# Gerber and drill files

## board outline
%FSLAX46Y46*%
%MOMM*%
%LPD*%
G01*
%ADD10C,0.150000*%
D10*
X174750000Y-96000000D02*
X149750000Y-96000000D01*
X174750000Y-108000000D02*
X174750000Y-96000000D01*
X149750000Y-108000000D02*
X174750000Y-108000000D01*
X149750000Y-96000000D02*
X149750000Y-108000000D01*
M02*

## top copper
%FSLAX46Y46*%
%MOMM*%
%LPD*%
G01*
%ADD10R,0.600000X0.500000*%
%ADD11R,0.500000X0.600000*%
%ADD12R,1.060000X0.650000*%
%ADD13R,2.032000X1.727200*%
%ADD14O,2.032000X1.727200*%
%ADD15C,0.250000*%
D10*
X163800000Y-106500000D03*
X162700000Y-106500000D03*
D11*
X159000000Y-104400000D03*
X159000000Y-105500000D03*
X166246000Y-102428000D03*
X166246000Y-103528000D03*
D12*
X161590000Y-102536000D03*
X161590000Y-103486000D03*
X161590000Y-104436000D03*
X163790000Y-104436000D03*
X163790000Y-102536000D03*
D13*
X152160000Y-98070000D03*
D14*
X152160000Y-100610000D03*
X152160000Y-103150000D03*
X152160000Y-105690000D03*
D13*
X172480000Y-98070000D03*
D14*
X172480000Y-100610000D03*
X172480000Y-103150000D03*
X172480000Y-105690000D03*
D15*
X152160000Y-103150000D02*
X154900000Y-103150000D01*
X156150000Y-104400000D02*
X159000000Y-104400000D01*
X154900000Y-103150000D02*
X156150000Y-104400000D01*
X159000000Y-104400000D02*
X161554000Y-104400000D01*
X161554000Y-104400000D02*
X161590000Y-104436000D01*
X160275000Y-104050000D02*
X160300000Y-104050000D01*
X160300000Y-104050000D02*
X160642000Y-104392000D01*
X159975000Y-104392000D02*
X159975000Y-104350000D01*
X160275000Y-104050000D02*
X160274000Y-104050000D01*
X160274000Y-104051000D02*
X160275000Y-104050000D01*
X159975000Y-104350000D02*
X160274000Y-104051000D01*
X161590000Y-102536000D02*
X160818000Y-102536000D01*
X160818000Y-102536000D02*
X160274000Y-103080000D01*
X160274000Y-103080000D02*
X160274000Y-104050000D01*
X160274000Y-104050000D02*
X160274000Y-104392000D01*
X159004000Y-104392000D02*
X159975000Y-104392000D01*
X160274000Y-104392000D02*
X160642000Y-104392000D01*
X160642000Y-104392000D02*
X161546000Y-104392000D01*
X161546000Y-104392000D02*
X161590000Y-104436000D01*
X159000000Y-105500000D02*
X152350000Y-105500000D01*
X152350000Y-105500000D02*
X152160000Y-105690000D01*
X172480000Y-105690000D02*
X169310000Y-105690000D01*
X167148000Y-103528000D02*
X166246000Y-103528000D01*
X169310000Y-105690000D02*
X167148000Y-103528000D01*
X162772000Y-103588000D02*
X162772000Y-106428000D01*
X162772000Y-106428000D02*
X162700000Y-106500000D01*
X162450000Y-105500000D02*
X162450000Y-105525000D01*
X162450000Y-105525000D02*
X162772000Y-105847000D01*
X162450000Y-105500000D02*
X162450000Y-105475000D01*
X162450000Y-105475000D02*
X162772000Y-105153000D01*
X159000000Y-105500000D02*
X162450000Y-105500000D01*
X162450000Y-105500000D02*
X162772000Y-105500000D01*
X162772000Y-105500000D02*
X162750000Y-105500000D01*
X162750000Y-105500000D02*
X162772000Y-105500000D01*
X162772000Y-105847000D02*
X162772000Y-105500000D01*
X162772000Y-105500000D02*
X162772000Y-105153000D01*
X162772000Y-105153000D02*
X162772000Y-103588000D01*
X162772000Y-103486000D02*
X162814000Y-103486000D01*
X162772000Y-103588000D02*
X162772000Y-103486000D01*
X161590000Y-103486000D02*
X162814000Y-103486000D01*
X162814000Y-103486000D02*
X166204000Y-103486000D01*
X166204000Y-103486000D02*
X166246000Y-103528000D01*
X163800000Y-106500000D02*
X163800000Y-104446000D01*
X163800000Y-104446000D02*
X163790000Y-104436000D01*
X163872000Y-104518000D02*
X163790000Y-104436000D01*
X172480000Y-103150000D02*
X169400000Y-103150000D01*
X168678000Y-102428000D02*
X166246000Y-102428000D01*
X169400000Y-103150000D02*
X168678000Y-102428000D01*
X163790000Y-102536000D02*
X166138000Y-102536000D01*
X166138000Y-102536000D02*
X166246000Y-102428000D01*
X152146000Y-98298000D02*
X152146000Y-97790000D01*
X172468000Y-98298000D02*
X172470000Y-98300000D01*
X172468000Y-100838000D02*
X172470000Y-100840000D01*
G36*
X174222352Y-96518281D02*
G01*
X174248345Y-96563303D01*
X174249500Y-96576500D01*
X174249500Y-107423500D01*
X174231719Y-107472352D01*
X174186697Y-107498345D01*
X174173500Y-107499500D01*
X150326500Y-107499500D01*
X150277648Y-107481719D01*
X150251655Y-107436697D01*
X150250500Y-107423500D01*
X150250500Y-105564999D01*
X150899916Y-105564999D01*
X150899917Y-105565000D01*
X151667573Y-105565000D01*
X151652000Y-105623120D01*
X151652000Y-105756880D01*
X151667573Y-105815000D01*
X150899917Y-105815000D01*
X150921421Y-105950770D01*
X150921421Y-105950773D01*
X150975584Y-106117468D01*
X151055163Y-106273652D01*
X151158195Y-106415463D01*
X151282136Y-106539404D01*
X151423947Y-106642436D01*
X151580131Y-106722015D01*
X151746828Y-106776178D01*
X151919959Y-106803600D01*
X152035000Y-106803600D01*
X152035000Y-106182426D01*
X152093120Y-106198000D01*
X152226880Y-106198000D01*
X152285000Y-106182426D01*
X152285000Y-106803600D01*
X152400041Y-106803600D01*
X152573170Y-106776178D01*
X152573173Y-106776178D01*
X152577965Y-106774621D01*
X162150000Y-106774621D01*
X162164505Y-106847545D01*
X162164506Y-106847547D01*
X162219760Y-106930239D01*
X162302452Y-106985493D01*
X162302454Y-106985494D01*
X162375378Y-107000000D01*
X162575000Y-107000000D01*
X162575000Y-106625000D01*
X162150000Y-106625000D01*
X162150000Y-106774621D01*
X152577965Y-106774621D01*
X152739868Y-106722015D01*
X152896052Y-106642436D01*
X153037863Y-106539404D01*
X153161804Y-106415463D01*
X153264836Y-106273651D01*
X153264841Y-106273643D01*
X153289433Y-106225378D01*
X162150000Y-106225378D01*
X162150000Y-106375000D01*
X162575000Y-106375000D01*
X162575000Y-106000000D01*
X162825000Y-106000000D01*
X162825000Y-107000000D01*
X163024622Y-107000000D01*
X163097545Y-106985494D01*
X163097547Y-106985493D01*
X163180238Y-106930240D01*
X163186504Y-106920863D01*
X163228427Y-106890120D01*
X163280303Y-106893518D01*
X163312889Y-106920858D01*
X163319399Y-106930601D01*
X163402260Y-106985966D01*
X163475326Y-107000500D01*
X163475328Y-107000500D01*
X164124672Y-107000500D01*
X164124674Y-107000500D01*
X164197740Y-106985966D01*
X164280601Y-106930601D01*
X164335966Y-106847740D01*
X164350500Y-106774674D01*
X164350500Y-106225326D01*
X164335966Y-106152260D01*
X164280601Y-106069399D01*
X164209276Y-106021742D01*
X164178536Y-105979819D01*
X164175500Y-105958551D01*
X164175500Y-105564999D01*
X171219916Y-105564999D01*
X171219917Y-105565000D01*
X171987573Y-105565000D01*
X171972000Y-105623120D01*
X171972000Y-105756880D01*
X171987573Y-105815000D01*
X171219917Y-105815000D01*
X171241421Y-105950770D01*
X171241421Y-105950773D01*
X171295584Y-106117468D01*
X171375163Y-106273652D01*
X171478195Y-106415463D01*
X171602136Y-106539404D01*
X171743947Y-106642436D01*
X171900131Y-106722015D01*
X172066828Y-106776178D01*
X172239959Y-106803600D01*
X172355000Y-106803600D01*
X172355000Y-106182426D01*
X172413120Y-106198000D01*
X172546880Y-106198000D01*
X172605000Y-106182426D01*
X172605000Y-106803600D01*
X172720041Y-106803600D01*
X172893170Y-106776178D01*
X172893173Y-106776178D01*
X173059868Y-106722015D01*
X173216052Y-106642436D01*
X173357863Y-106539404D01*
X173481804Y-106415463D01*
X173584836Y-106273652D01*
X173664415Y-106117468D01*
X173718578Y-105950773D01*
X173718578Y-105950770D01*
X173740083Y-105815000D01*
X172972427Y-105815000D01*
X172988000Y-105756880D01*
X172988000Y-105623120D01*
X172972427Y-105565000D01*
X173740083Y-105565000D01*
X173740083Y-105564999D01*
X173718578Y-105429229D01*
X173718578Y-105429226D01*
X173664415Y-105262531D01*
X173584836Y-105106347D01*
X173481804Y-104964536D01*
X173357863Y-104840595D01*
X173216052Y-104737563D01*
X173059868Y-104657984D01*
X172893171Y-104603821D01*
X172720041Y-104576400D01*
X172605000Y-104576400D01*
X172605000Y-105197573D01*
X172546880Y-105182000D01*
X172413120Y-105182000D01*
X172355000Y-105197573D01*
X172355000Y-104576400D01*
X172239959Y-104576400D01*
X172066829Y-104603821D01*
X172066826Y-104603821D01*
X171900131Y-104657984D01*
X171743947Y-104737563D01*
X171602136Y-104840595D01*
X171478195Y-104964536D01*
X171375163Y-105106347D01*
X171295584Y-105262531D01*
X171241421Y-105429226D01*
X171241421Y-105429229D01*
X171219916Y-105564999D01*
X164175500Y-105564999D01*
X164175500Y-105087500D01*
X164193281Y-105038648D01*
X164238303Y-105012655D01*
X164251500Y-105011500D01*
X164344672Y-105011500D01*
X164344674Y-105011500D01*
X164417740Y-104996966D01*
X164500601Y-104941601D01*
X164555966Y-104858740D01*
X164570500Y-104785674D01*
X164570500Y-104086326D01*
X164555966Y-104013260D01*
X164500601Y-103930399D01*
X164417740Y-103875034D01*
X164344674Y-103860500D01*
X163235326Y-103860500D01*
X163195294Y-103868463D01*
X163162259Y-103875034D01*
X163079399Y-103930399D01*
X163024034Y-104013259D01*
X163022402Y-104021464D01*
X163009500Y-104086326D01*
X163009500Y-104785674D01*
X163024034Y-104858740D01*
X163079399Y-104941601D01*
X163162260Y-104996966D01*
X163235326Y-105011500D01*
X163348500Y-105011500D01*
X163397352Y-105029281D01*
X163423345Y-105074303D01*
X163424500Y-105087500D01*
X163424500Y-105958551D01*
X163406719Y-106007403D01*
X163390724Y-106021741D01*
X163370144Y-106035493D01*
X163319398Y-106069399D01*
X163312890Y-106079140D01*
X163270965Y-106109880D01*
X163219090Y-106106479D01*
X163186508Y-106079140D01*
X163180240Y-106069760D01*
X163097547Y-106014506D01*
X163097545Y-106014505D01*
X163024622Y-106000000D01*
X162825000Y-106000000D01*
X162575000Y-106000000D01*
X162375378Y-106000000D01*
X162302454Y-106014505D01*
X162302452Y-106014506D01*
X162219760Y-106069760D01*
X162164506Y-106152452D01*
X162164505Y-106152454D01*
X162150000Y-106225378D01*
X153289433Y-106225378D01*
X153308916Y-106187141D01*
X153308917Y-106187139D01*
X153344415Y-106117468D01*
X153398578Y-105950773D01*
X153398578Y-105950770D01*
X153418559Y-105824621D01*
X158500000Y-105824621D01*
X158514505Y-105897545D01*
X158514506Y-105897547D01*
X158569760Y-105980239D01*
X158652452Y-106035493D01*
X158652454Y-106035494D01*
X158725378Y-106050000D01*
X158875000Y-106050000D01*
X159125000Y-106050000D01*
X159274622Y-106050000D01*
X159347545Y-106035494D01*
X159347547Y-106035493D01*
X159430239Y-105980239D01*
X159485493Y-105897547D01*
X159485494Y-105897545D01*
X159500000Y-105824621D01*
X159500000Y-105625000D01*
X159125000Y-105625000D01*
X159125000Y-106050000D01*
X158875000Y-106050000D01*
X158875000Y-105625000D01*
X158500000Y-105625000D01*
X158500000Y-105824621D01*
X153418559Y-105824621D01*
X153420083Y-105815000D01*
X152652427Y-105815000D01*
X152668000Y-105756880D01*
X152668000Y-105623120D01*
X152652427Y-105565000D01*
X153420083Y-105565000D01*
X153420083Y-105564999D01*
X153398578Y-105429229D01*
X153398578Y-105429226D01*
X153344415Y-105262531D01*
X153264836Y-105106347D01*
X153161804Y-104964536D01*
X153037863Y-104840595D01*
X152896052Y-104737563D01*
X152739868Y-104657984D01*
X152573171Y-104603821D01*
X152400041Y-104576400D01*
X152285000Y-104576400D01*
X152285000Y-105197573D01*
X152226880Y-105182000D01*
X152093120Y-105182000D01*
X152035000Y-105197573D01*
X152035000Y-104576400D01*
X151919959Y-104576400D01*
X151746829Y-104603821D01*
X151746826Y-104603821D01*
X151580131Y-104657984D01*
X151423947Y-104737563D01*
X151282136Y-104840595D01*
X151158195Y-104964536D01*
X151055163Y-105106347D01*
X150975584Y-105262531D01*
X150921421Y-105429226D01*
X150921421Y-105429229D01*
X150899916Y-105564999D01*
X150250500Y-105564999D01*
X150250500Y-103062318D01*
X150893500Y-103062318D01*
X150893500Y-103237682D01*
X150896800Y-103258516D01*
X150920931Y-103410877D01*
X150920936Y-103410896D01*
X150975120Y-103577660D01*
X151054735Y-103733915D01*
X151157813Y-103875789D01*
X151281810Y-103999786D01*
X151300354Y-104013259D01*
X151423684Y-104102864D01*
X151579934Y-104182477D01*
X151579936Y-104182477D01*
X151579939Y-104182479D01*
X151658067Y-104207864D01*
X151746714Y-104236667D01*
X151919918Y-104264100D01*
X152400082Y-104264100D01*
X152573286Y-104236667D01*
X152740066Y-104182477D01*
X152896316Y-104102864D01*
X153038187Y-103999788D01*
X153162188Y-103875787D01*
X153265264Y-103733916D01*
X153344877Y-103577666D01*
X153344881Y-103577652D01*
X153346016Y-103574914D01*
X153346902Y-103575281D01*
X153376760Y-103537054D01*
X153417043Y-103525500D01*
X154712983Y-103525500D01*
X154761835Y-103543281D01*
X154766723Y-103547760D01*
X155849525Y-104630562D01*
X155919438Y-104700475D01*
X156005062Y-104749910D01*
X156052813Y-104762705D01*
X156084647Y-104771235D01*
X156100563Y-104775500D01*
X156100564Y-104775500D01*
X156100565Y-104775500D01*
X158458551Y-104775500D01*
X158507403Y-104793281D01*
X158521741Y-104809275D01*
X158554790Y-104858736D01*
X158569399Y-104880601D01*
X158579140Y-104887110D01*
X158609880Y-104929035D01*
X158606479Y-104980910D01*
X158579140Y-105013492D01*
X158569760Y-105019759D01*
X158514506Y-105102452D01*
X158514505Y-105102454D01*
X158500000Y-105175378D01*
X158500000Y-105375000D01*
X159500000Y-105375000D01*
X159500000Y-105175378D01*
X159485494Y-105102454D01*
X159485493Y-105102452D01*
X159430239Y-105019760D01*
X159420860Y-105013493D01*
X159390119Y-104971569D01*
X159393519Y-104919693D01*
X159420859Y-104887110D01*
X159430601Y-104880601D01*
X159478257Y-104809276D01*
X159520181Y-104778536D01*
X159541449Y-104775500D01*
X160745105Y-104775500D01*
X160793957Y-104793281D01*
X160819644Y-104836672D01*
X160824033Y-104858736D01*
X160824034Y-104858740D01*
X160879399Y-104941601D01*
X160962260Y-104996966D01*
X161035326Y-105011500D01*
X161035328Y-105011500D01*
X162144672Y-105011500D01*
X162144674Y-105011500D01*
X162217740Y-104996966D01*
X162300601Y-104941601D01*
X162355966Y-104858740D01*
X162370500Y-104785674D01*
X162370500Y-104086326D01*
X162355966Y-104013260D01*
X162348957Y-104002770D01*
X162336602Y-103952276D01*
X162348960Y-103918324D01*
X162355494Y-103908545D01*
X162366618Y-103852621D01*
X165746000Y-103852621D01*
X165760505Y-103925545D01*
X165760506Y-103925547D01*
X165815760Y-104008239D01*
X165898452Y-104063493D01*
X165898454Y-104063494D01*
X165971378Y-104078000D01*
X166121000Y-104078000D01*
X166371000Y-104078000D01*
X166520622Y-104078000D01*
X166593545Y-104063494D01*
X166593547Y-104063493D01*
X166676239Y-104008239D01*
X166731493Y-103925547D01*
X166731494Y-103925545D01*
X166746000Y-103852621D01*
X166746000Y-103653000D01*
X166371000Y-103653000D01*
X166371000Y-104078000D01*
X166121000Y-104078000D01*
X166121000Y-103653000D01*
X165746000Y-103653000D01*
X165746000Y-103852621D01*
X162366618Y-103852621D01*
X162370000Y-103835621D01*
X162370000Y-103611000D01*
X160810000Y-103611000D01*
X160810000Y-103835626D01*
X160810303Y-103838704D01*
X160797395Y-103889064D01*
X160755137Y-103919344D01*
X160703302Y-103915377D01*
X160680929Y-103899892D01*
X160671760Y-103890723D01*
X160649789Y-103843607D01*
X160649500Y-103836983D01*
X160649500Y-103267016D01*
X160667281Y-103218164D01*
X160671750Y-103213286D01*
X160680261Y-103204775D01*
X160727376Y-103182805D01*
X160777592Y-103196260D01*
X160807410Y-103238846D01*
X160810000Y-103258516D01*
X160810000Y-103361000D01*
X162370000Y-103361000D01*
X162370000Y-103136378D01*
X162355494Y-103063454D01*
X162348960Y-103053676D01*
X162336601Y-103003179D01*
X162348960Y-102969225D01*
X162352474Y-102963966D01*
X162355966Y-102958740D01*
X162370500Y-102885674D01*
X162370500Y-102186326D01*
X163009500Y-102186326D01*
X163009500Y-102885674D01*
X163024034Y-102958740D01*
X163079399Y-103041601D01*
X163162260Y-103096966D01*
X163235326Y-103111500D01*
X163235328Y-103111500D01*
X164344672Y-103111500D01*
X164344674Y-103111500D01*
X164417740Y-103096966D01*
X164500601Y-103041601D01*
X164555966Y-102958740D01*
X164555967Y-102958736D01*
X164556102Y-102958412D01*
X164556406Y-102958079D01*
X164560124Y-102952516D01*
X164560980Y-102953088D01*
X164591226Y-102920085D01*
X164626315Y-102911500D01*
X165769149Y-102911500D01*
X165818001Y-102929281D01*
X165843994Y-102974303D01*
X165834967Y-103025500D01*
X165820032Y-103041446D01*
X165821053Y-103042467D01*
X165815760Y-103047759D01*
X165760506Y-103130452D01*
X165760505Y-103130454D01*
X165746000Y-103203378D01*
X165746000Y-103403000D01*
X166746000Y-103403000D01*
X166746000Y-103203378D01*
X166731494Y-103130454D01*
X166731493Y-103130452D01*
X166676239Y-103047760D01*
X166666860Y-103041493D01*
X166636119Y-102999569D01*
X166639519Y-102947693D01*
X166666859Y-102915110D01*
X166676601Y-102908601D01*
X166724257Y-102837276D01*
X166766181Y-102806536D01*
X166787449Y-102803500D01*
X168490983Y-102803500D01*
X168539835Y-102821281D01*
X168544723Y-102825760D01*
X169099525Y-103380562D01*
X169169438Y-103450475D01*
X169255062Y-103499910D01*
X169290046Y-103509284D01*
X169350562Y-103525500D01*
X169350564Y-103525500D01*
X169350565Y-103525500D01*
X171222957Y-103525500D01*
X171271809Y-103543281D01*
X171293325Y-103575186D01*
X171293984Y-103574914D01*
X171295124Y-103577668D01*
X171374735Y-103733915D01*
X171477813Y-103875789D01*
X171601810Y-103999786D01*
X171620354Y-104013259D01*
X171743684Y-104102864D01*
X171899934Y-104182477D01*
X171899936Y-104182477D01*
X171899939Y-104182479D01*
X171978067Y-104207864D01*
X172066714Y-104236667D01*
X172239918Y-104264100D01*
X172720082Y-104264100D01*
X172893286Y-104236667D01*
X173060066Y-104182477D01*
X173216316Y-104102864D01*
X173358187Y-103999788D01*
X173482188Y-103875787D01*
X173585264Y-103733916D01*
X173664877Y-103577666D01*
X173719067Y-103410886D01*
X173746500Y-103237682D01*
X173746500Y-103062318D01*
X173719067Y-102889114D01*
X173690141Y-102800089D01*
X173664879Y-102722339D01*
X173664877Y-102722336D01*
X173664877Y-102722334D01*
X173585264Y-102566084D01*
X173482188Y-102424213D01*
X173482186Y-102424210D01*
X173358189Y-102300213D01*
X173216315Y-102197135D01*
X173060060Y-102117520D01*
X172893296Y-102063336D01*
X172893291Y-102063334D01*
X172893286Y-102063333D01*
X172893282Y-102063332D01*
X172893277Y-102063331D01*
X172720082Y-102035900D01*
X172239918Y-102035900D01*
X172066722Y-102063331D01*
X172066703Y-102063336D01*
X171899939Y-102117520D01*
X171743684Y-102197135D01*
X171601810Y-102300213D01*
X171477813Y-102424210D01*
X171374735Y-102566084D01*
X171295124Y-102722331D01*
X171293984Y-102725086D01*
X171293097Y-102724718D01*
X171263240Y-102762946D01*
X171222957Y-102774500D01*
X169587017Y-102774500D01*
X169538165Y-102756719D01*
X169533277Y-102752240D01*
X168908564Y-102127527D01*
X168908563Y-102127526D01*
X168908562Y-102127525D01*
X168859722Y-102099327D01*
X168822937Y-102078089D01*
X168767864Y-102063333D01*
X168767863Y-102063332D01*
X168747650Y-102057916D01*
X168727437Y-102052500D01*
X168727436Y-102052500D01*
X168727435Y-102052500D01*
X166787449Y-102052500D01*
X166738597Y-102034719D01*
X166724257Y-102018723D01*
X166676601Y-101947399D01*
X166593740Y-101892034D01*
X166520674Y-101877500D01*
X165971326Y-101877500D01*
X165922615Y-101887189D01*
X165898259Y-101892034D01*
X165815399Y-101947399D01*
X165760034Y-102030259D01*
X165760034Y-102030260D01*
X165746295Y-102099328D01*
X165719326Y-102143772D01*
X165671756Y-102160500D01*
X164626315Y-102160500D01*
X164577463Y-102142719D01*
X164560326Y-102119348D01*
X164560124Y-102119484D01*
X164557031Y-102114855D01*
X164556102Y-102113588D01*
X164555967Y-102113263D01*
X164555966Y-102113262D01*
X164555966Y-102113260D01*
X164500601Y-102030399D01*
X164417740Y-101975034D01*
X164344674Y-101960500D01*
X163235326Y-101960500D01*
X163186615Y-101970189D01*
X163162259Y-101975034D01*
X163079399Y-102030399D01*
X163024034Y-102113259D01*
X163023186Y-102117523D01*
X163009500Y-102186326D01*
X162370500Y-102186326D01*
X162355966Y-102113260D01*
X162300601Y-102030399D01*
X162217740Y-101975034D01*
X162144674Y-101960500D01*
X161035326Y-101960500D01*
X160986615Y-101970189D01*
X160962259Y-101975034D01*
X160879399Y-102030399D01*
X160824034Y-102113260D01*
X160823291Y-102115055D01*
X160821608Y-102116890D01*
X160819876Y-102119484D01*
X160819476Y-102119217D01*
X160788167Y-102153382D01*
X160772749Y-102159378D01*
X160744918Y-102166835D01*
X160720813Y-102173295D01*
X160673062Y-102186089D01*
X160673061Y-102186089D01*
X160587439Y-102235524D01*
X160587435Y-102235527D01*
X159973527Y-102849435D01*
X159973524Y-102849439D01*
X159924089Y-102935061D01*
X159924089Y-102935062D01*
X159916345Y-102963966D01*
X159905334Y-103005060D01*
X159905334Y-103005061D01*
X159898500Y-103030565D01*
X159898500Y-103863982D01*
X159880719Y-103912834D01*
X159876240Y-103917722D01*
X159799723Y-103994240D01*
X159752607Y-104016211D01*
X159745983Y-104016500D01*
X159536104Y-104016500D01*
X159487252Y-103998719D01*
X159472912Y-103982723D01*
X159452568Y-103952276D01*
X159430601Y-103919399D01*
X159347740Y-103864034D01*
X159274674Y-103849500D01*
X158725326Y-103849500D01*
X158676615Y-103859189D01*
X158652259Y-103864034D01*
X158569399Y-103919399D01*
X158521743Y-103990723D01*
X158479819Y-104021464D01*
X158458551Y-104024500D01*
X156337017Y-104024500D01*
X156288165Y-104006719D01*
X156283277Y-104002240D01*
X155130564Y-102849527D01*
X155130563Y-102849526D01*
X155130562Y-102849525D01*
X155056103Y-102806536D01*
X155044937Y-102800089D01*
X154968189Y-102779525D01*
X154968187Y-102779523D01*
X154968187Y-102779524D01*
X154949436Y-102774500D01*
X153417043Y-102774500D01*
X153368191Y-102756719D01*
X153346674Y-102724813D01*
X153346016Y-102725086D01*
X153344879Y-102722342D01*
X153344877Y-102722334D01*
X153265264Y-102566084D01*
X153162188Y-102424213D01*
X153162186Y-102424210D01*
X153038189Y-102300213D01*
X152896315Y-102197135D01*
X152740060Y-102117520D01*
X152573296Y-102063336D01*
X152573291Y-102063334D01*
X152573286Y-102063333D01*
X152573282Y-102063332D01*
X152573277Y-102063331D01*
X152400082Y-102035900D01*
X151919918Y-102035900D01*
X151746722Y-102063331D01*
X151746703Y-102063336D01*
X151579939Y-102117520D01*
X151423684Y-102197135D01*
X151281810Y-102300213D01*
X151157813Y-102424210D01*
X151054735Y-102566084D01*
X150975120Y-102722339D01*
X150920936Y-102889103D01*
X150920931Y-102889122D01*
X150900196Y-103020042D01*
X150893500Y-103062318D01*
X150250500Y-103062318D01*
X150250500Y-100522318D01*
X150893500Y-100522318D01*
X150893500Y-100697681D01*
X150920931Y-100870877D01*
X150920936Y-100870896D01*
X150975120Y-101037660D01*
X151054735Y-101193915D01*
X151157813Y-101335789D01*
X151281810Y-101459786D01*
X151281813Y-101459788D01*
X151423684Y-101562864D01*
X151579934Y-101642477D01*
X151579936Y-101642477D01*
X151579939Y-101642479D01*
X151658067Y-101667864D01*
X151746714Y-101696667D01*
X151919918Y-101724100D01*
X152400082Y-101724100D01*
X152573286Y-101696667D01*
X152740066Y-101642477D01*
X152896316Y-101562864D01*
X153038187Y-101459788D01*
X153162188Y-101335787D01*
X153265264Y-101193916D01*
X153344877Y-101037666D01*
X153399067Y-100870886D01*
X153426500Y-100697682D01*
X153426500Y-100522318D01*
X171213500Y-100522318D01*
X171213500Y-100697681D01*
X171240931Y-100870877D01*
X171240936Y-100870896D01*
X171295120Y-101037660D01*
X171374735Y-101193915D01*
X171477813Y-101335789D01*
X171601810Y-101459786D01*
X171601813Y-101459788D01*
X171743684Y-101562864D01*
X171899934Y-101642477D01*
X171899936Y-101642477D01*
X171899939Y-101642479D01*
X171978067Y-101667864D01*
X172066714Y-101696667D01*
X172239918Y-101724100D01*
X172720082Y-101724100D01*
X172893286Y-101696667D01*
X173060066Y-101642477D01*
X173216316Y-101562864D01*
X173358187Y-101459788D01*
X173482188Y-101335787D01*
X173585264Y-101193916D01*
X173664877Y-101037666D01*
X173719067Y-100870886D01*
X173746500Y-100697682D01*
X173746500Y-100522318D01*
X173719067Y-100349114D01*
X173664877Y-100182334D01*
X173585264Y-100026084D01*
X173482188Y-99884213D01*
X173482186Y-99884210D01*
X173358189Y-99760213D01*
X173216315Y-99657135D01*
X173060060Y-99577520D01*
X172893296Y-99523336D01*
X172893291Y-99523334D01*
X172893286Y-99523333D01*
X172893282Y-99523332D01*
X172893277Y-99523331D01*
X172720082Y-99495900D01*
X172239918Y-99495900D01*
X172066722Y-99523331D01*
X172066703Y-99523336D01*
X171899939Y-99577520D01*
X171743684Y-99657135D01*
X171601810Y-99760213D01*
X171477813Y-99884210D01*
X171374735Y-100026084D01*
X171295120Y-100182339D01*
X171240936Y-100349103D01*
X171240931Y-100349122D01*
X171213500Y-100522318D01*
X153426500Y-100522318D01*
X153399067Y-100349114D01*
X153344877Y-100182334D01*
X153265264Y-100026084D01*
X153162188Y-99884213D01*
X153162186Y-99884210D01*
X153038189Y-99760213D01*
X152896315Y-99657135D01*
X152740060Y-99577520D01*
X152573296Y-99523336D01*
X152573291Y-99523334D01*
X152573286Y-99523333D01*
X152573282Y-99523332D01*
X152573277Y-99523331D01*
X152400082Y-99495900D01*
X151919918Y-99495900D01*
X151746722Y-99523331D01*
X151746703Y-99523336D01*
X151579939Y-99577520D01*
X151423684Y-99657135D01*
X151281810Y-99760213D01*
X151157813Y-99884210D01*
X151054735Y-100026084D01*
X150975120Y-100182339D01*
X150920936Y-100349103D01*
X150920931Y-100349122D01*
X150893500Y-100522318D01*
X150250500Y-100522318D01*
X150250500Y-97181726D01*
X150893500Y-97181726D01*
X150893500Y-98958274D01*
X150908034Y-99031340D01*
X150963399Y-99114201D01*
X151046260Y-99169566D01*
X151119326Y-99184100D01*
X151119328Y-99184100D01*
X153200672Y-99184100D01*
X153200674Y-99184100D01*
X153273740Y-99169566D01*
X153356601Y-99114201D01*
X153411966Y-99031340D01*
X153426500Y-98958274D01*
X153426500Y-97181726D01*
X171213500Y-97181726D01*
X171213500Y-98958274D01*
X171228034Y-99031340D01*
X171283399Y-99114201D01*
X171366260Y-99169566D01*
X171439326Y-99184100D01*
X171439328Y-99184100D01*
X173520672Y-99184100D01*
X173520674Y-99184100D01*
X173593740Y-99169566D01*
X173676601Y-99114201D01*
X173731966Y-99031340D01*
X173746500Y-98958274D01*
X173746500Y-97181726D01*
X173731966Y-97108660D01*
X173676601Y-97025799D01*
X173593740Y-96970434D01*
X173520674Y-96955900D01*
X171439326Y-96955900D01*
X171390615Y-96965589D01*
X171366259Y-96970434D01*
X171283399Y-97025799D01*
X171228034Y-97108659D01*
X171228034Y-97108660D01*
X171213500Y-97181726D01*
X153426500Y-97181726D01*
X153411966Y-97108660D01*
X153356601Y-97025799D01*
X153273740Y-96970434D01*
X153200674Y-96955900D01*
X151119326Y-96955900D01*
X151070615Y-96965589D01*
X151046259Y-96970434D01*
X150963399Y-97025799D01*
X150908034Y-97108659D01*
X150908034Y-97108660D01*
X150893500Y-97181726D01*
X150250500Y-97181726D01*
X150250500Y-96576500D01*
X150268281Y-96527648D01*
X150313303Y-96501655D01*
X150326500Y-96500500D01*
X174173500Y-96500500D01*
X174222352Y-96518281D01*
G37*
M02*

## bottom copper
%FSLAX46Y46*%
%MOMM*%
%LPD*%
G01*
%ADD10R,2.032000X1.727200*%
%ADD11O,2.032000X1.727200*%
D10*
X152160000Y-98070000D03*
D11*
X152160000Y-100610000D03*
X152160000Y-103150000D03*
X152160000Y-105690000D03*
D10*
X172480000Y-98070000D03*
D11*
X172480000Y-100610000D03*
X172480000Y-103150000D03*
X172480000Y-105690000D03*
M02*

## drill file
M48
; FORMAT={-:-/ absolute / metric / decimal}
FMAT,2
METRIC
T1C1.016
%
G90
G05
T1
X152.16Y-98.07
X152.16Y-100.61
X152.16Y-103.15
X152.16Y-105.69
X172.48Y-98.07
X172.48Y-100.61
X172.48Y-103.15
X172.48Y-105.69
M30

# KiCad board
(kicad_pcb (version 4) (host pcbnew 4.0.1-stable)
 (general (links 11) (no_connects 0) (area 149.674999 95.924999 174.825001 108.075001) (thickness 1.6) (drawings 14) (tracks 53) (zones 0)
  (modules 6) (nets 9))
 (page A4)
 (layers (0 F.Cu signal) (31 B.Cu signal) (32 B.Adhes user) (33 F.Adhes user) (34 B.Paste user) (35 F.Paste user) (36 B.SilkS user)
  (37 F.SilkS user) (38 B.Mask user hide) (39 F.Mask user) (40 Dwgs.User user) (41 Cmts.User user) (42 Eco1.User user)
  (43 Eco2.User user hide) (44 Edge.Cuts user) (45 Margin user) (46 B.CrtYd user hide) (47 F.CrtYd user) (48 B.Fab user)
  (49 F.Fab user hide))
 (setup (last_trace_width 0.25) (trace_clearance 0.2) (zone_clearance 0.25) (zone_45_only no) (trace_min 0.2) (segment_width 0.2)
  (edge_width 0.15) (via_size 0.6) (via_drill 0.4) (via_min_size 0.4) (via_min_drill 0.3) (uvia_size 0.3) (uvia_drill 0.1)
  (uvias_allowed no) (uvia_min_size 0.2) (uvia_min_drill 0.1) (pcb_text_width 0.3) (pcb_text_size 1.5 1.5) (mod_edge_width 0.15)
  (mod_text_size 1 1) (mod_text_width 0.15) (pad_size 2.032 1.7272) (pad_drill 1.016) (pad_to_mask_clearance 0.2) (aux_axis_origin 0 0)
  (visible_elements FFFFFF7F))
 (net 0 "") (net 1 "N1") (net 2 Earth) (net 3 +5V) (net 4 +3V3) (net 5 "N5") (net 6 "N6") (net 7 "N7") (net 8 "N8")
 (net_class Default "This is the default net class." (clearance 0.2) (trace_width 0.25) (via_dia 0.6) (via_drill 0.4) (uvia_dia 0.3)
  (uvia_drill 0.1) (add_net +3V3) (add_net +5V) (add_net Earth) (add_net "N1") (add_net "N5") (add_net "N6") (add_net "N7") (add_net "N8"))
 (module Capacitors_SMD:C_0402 (layer F.Cu) (at 163.25 106.5 180)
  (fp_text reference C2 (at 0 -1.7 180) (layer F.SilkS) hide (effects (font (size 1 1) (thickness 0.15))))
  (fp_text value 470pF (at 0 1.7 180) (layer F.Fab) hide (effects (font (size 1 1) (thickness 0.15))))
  (pad 1 smd rect (at -0.55 0 180) (size 0.6 0.5) (layers F.Cu F.Paste F.Mask) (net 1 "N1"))
  (pad 2 smd rect (at 0.55 0 180) (size 0.6 0.5) (layers F.Cu F.Paste F.Mask) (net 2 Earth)))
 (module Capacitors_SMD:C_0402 (layer F.Cu) (at 159 104.95 270)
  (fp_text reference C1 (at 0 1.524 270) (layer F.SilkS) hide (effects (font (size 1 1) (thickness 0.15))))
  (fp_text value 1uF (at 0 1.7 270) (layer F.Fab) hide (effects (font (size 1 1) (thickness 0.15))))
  (pad 1 smd rect (at -0.55 0 270) (size 0.6 0.5) (layers F.Cu F.Paste F.Mask) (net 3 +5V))
  (pad 2 smd rect (at 0.55 0 270) (size 0.6 0.5) (layers F.Cu F.Paste F.Mask) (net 2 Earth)))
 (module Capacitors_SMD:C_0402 (layer F.Cu) (at 166.246 102.978 270)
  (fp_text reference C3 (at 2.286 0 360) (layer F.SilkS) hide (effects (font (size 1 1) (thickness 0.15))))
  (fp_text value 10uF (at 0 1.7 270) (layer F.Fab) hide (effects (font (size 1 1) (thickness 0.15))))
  (pad 1 smd rect (at -0.55 0 270) (size 0.6 0.5) (layers F.Cu F.Paste F.Mask) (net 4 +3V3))
  (pad 2 smd rect (at 0.55 0 270) (size 0.6 0.5) (layers F.Cu F.Paste F.Mask) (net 2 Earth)))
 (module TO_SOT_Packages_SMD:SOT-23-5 (layer F.Cu) (at 162.69 103.486)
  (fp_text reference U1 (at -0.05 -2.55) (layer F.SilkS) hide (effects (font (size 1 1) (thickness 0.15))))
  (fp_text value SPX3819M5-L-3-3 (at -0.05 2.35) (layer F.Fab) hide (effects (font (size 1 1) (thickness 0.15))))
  (pad 1 smd rect (at -1.1 -0.95) (size 1.06 0.65) (layers F.Cu F.Paste F.Mask) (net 3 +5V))
  (pad 2 smd rect (at -1.1 0) (size 1.06 0.65) (layers F.Cu F.Paste F.Mask) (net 2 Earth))
  (pad 3 smd rect (at -1.1 0.95) (size 1.06 0.65) (layers F.Cu F.Paste F.Mask) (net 3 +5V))
  (pad 4 smd rect (at 1.1 0.95) (size 1.06 0.65) (layers F.Cu F.Paste F.Mask) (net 1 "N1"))
  (pad 5 smd rect (at 1.1 -0.95) (size 1.06 0.65) (layers F.Cu F.Paste F.Mask) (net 4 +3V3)))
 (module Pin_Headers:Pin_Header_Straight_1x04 (layer F.Cu) (at 152.16 98.07)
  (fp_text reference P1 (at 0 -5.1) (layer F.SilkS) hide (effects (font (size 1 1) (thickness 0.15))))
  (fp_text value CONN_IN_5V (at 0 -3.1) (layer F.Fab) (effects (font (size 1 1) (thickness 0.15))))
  (pad 1 thru_hole rect (at 0 0) (size 2.032 1.7272) (drill 1.016) (layers *.Cu *.Mask F.SilkS) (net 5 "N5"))
  (pad 2 thru_hole oval (at 0 2.54) (size 2.032 1.7272) (drill 1.016) (layers *.Cu *.Mask F.SilkS) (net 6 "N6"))
  (pad 3 thru_hole oval (at 0 5.08) (size 2.032 1.7272) (drill 1.016) (layers *.Cu *.Mask F.SilkS) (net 3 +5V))
  (pad 4 thru_hole oval (at 0 7.62) (size 2.032 1.7272) (drill 1.016) (layers *.Cu *.Mask F.SilkS) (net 2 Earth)))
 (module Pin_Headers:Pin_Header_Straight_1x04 (layer F.Cu) (at 172.48 98.07)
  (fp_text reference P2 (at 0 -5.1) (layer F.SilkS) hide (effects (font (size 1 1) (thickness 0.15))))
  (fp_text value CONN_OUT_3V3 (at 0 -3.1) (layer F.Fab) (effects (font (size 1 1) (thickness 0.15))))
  (pad 1 thru_hole rect (at 0 0) (size 2.032 1.7272) (drill 1.016) (layers *.Cu *.Mask F.SilkS) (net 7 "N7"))
  (pad 2 thru_hole oval (at 0 2.54) (size 2.032 1.7272) (drill 1.016) (layers *.Cu *.Mask F.SilkS) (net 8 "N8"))
  (pad 3 thru_hole oval (at 0 5.08) (size 2.032 1.7272) (drill 1.016) (layers *.Cu *.Mask F.SilkS) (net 4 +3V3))
  (pad 4 thru_hole oval (at 0 7.62) (size 2.032 1.7272) (drill 1.016) (layers *.Cu *.Mask F.SilkS) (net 2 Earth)))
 (gr_line (start 174.75 96) (end 149.75 96) (angle 90) (layer Edge.Cuts) (width 0.15))
 (gr_line (start 174.75 108) (end 174.75 96) (angle 90) (layer Edge.Cuts) (width 0.15))
 (gr_line (start 149.75 108) (end 174.75 108) (angle 90) (layer Edge.Cuts) (width 0.15))
 (gr_line (start 149.75 96) (end 149.75 108) (angle 90) (layer Edge.Cuts) (width 0.15))
 (segment (start 152.16 103.15) (end 154.9 103.15) (width 0.25) (layer F.Cu) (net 3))
 (segment (start 156.15 104.4) (end 159 104.4) (width 0.25) (layer F.Cu) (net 3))
 (segment (start 154.9 103.15) (end 156.15 104.4) (width 0.25) (layer F.Cu) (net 3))
 (segment (start 159 104.4) (end 161.554 104.4) (width 0.25) (layer F.Cu) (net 3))
 (segment (start 161.554 104.4) (end 161.59 104.436) (width 0.25) (layer F.Cu) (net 3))
 (segment (start 160.275 104.05) (end 160.3 104.05) (width 0.25) (layer F.Cu) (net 3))
 (segment (start 160.3 104.05) (end 160.642 104.392) (width 0.25) (layer F.Cu) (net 3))
 (segment (start 159.975 104.392) (end 159.975 104.35) (width 0.25) (layer F.Cu) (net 3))
 (segment (start 160.275 104.05) (end 160.274 104.05) (width 0.25) (layer F.Cu) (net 3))
 (segment (start 160.274 104.051) (end 160.275 104.05) (width 0.25) (layer F.Cu) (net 3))
 (segment (start 159.975 104.35) (end 160.274 104.051) (width 0.25) (layer F.Cu) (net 3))
 (segment (start 161.59 102.536) (end 160.818 102.536) (width 0.25) (layer F.Cu) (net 3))
 (segment (start 160.818 102.536) (end 160.274 103.08) (width 0.25) (layer F.Cu) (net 3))
 (segment (start 160.274 103.08) (end 160.274 104.05) (width 0.25) (layer F.Cu) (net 3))
 (segment (start 160.274 104.05) (end 160.274 104.392) (width 0.25) (layer F.Cu) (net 3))
 (segment (start 159.004 104.392) (end 159.975 104.392) (width 0.25) (layer F.Cu) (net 3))
 (segment (start 160.274 104.392) (end 160.642 104.392) (width 0.25) (layer F.Cu) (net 3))
 (segment (start 160.642 104.392) (end 161.546 104.392) (width 0.25) (layer F.Cu) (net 3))
 (segment (start 161.546 104.392) (end 161.59 104.436) (width 0.25) (layer F.Cu) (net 3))
 (segment (start 159 105.5) (end 152.35 105.5) (width 0.25) (layer F.Cu) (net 2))
 (segment (start 152.35 105.5) (end 152.16 105.69) (width 0.25) (layer F.Cu) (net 2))
 (segment (start 172.48 105.69) (end 169.31 105.69) (width 0.25) (layer F.Cu) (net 2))
 (segment (start 167.148 103.528) (end 166.246 103.528) (width 0.25) (layer F.Cu) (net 2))
 (segment (start 169.31 105.69) (end 167.148 103.528) (width 0.25) (layer F.Cu) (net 2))
 (segment (start 162.772 103.588) (end 162.772 106.428) (width 0.25) (layer F.Cu) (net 2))
 (segment (start 162.772 106.428) (end 162.7 106.5) (width 0.25) (layer F.Cu) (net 2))
 (segment (start 162.45 105.5) (end 162.45 105.525) (width 0.25) (layer F.Cu) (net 2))
 (segment (start 162.45 105.525) (end 162.772 105.847) (width 0.25) (layer F.Cu) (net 2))
 (segment (start 162.45 105.5) (end 162.45 105.475) (width 0.25) (layer F.Cu) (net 2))
 (segment (start 162.45 105.475) (end 162.772 105.153) (width 0.25) (layer F.Cu) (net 2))
 (segment (start 159 105.5) (end 162.45 105.5) (width 0.25) (layer F.Cu) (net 2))
 (segment (start 162.45 105.5) (end 162.772 105.5) (width 0.25) (layer F.Cu) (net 2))
 (segment (start 162.772 105.5) (end 162.75 105.5) (width 0.25) (layer F.Cu) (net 2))
 (segment (start 162.75 105.5) (end 162.772 105.5) (width 0.25) (layer F.Cu) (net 2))
 (segment (start 162.772 105.847) (end 162.772 105.5) (width 0.25) (layer F.Cu) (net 2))
 (segment (start 162.772 105.5) (end 162.772 105.153) (width 0.25) (layer F.Cu) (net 2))
 (segment (start 162.772 105.153) (end 162.772 103.588) (width 0.25) (layer F.Cu) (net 2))
 (segment (start 162.772 103.486) (end 162.814 103.486) (width 0.25) (layer F.Cu) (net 2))
 (segment (start 162.772 103.588) (end 162.772 103.486) (width 0.25) (layer F.Cu) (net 2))
 (segment (start 161.59 103.486) (end 162.814 103.486) (width 0.25) (layer F.Cu) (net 2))
 (segment (start 162.814 103.486) (end 166.204 103.486) (width 0.25) (layer F.Cu) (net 2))
 (segment (start 166.204 103.486) (end 166.246 103.528) (width 0.25) (layer F.Cu) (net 2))
 (segment (start 163.8 106.5) (end 163.8 104.446) (width 0.25) (layer F.Cu) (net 1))
 (segment (start 163.8 104.446) (end 163.79 104.436) (width 0.25) (layer F.Cu) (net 1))
 (segment (start 163.872 104.518) (end 163.79 104.436) (width 0.25) (layer F.Cu) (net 1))
 (segment (start 172.48 103.15) (end 169.4 103.15) (width 0.25) (layer F.Cu) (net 4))
 (segment (start 168.678 102.428) (end 166.246 102.428) (width 0.25) (layer F.Cu) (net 4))
 (segment (start 169.4 103.15) (end 168.678 102.428) (width 0.25) (layer F.Cu) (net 4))
 (segment (start 163.79 102.536) (end 166.138 102.536) (width 0.25) (layer F.Cu) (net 4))
 (segment (start 166.138 102.536) (end 166.246 102.428) (width 0.25) (layer F.Cu) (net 4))
 (segment (start 152.146 98.298) (end 152.146 97.79) (width 0.25) (layer F.Cu) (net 5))
 (segment (start 172.468 98.298) (end 172.47 98.3) (width 0.25) (layer F.Cu) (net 7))
 (segment (start 172.468 100.838) (end 172.47 100.84) (width 0.25) (layer F.Cu) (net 8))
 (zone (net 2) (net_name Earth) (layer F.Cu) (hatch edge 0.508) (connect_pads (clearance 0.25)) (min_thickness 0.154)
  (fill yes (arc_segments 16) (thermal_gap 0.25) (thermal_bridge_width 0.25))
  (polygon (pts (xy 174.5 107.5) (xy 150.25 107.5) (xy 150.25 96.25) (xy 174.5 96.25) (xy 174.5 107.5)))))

